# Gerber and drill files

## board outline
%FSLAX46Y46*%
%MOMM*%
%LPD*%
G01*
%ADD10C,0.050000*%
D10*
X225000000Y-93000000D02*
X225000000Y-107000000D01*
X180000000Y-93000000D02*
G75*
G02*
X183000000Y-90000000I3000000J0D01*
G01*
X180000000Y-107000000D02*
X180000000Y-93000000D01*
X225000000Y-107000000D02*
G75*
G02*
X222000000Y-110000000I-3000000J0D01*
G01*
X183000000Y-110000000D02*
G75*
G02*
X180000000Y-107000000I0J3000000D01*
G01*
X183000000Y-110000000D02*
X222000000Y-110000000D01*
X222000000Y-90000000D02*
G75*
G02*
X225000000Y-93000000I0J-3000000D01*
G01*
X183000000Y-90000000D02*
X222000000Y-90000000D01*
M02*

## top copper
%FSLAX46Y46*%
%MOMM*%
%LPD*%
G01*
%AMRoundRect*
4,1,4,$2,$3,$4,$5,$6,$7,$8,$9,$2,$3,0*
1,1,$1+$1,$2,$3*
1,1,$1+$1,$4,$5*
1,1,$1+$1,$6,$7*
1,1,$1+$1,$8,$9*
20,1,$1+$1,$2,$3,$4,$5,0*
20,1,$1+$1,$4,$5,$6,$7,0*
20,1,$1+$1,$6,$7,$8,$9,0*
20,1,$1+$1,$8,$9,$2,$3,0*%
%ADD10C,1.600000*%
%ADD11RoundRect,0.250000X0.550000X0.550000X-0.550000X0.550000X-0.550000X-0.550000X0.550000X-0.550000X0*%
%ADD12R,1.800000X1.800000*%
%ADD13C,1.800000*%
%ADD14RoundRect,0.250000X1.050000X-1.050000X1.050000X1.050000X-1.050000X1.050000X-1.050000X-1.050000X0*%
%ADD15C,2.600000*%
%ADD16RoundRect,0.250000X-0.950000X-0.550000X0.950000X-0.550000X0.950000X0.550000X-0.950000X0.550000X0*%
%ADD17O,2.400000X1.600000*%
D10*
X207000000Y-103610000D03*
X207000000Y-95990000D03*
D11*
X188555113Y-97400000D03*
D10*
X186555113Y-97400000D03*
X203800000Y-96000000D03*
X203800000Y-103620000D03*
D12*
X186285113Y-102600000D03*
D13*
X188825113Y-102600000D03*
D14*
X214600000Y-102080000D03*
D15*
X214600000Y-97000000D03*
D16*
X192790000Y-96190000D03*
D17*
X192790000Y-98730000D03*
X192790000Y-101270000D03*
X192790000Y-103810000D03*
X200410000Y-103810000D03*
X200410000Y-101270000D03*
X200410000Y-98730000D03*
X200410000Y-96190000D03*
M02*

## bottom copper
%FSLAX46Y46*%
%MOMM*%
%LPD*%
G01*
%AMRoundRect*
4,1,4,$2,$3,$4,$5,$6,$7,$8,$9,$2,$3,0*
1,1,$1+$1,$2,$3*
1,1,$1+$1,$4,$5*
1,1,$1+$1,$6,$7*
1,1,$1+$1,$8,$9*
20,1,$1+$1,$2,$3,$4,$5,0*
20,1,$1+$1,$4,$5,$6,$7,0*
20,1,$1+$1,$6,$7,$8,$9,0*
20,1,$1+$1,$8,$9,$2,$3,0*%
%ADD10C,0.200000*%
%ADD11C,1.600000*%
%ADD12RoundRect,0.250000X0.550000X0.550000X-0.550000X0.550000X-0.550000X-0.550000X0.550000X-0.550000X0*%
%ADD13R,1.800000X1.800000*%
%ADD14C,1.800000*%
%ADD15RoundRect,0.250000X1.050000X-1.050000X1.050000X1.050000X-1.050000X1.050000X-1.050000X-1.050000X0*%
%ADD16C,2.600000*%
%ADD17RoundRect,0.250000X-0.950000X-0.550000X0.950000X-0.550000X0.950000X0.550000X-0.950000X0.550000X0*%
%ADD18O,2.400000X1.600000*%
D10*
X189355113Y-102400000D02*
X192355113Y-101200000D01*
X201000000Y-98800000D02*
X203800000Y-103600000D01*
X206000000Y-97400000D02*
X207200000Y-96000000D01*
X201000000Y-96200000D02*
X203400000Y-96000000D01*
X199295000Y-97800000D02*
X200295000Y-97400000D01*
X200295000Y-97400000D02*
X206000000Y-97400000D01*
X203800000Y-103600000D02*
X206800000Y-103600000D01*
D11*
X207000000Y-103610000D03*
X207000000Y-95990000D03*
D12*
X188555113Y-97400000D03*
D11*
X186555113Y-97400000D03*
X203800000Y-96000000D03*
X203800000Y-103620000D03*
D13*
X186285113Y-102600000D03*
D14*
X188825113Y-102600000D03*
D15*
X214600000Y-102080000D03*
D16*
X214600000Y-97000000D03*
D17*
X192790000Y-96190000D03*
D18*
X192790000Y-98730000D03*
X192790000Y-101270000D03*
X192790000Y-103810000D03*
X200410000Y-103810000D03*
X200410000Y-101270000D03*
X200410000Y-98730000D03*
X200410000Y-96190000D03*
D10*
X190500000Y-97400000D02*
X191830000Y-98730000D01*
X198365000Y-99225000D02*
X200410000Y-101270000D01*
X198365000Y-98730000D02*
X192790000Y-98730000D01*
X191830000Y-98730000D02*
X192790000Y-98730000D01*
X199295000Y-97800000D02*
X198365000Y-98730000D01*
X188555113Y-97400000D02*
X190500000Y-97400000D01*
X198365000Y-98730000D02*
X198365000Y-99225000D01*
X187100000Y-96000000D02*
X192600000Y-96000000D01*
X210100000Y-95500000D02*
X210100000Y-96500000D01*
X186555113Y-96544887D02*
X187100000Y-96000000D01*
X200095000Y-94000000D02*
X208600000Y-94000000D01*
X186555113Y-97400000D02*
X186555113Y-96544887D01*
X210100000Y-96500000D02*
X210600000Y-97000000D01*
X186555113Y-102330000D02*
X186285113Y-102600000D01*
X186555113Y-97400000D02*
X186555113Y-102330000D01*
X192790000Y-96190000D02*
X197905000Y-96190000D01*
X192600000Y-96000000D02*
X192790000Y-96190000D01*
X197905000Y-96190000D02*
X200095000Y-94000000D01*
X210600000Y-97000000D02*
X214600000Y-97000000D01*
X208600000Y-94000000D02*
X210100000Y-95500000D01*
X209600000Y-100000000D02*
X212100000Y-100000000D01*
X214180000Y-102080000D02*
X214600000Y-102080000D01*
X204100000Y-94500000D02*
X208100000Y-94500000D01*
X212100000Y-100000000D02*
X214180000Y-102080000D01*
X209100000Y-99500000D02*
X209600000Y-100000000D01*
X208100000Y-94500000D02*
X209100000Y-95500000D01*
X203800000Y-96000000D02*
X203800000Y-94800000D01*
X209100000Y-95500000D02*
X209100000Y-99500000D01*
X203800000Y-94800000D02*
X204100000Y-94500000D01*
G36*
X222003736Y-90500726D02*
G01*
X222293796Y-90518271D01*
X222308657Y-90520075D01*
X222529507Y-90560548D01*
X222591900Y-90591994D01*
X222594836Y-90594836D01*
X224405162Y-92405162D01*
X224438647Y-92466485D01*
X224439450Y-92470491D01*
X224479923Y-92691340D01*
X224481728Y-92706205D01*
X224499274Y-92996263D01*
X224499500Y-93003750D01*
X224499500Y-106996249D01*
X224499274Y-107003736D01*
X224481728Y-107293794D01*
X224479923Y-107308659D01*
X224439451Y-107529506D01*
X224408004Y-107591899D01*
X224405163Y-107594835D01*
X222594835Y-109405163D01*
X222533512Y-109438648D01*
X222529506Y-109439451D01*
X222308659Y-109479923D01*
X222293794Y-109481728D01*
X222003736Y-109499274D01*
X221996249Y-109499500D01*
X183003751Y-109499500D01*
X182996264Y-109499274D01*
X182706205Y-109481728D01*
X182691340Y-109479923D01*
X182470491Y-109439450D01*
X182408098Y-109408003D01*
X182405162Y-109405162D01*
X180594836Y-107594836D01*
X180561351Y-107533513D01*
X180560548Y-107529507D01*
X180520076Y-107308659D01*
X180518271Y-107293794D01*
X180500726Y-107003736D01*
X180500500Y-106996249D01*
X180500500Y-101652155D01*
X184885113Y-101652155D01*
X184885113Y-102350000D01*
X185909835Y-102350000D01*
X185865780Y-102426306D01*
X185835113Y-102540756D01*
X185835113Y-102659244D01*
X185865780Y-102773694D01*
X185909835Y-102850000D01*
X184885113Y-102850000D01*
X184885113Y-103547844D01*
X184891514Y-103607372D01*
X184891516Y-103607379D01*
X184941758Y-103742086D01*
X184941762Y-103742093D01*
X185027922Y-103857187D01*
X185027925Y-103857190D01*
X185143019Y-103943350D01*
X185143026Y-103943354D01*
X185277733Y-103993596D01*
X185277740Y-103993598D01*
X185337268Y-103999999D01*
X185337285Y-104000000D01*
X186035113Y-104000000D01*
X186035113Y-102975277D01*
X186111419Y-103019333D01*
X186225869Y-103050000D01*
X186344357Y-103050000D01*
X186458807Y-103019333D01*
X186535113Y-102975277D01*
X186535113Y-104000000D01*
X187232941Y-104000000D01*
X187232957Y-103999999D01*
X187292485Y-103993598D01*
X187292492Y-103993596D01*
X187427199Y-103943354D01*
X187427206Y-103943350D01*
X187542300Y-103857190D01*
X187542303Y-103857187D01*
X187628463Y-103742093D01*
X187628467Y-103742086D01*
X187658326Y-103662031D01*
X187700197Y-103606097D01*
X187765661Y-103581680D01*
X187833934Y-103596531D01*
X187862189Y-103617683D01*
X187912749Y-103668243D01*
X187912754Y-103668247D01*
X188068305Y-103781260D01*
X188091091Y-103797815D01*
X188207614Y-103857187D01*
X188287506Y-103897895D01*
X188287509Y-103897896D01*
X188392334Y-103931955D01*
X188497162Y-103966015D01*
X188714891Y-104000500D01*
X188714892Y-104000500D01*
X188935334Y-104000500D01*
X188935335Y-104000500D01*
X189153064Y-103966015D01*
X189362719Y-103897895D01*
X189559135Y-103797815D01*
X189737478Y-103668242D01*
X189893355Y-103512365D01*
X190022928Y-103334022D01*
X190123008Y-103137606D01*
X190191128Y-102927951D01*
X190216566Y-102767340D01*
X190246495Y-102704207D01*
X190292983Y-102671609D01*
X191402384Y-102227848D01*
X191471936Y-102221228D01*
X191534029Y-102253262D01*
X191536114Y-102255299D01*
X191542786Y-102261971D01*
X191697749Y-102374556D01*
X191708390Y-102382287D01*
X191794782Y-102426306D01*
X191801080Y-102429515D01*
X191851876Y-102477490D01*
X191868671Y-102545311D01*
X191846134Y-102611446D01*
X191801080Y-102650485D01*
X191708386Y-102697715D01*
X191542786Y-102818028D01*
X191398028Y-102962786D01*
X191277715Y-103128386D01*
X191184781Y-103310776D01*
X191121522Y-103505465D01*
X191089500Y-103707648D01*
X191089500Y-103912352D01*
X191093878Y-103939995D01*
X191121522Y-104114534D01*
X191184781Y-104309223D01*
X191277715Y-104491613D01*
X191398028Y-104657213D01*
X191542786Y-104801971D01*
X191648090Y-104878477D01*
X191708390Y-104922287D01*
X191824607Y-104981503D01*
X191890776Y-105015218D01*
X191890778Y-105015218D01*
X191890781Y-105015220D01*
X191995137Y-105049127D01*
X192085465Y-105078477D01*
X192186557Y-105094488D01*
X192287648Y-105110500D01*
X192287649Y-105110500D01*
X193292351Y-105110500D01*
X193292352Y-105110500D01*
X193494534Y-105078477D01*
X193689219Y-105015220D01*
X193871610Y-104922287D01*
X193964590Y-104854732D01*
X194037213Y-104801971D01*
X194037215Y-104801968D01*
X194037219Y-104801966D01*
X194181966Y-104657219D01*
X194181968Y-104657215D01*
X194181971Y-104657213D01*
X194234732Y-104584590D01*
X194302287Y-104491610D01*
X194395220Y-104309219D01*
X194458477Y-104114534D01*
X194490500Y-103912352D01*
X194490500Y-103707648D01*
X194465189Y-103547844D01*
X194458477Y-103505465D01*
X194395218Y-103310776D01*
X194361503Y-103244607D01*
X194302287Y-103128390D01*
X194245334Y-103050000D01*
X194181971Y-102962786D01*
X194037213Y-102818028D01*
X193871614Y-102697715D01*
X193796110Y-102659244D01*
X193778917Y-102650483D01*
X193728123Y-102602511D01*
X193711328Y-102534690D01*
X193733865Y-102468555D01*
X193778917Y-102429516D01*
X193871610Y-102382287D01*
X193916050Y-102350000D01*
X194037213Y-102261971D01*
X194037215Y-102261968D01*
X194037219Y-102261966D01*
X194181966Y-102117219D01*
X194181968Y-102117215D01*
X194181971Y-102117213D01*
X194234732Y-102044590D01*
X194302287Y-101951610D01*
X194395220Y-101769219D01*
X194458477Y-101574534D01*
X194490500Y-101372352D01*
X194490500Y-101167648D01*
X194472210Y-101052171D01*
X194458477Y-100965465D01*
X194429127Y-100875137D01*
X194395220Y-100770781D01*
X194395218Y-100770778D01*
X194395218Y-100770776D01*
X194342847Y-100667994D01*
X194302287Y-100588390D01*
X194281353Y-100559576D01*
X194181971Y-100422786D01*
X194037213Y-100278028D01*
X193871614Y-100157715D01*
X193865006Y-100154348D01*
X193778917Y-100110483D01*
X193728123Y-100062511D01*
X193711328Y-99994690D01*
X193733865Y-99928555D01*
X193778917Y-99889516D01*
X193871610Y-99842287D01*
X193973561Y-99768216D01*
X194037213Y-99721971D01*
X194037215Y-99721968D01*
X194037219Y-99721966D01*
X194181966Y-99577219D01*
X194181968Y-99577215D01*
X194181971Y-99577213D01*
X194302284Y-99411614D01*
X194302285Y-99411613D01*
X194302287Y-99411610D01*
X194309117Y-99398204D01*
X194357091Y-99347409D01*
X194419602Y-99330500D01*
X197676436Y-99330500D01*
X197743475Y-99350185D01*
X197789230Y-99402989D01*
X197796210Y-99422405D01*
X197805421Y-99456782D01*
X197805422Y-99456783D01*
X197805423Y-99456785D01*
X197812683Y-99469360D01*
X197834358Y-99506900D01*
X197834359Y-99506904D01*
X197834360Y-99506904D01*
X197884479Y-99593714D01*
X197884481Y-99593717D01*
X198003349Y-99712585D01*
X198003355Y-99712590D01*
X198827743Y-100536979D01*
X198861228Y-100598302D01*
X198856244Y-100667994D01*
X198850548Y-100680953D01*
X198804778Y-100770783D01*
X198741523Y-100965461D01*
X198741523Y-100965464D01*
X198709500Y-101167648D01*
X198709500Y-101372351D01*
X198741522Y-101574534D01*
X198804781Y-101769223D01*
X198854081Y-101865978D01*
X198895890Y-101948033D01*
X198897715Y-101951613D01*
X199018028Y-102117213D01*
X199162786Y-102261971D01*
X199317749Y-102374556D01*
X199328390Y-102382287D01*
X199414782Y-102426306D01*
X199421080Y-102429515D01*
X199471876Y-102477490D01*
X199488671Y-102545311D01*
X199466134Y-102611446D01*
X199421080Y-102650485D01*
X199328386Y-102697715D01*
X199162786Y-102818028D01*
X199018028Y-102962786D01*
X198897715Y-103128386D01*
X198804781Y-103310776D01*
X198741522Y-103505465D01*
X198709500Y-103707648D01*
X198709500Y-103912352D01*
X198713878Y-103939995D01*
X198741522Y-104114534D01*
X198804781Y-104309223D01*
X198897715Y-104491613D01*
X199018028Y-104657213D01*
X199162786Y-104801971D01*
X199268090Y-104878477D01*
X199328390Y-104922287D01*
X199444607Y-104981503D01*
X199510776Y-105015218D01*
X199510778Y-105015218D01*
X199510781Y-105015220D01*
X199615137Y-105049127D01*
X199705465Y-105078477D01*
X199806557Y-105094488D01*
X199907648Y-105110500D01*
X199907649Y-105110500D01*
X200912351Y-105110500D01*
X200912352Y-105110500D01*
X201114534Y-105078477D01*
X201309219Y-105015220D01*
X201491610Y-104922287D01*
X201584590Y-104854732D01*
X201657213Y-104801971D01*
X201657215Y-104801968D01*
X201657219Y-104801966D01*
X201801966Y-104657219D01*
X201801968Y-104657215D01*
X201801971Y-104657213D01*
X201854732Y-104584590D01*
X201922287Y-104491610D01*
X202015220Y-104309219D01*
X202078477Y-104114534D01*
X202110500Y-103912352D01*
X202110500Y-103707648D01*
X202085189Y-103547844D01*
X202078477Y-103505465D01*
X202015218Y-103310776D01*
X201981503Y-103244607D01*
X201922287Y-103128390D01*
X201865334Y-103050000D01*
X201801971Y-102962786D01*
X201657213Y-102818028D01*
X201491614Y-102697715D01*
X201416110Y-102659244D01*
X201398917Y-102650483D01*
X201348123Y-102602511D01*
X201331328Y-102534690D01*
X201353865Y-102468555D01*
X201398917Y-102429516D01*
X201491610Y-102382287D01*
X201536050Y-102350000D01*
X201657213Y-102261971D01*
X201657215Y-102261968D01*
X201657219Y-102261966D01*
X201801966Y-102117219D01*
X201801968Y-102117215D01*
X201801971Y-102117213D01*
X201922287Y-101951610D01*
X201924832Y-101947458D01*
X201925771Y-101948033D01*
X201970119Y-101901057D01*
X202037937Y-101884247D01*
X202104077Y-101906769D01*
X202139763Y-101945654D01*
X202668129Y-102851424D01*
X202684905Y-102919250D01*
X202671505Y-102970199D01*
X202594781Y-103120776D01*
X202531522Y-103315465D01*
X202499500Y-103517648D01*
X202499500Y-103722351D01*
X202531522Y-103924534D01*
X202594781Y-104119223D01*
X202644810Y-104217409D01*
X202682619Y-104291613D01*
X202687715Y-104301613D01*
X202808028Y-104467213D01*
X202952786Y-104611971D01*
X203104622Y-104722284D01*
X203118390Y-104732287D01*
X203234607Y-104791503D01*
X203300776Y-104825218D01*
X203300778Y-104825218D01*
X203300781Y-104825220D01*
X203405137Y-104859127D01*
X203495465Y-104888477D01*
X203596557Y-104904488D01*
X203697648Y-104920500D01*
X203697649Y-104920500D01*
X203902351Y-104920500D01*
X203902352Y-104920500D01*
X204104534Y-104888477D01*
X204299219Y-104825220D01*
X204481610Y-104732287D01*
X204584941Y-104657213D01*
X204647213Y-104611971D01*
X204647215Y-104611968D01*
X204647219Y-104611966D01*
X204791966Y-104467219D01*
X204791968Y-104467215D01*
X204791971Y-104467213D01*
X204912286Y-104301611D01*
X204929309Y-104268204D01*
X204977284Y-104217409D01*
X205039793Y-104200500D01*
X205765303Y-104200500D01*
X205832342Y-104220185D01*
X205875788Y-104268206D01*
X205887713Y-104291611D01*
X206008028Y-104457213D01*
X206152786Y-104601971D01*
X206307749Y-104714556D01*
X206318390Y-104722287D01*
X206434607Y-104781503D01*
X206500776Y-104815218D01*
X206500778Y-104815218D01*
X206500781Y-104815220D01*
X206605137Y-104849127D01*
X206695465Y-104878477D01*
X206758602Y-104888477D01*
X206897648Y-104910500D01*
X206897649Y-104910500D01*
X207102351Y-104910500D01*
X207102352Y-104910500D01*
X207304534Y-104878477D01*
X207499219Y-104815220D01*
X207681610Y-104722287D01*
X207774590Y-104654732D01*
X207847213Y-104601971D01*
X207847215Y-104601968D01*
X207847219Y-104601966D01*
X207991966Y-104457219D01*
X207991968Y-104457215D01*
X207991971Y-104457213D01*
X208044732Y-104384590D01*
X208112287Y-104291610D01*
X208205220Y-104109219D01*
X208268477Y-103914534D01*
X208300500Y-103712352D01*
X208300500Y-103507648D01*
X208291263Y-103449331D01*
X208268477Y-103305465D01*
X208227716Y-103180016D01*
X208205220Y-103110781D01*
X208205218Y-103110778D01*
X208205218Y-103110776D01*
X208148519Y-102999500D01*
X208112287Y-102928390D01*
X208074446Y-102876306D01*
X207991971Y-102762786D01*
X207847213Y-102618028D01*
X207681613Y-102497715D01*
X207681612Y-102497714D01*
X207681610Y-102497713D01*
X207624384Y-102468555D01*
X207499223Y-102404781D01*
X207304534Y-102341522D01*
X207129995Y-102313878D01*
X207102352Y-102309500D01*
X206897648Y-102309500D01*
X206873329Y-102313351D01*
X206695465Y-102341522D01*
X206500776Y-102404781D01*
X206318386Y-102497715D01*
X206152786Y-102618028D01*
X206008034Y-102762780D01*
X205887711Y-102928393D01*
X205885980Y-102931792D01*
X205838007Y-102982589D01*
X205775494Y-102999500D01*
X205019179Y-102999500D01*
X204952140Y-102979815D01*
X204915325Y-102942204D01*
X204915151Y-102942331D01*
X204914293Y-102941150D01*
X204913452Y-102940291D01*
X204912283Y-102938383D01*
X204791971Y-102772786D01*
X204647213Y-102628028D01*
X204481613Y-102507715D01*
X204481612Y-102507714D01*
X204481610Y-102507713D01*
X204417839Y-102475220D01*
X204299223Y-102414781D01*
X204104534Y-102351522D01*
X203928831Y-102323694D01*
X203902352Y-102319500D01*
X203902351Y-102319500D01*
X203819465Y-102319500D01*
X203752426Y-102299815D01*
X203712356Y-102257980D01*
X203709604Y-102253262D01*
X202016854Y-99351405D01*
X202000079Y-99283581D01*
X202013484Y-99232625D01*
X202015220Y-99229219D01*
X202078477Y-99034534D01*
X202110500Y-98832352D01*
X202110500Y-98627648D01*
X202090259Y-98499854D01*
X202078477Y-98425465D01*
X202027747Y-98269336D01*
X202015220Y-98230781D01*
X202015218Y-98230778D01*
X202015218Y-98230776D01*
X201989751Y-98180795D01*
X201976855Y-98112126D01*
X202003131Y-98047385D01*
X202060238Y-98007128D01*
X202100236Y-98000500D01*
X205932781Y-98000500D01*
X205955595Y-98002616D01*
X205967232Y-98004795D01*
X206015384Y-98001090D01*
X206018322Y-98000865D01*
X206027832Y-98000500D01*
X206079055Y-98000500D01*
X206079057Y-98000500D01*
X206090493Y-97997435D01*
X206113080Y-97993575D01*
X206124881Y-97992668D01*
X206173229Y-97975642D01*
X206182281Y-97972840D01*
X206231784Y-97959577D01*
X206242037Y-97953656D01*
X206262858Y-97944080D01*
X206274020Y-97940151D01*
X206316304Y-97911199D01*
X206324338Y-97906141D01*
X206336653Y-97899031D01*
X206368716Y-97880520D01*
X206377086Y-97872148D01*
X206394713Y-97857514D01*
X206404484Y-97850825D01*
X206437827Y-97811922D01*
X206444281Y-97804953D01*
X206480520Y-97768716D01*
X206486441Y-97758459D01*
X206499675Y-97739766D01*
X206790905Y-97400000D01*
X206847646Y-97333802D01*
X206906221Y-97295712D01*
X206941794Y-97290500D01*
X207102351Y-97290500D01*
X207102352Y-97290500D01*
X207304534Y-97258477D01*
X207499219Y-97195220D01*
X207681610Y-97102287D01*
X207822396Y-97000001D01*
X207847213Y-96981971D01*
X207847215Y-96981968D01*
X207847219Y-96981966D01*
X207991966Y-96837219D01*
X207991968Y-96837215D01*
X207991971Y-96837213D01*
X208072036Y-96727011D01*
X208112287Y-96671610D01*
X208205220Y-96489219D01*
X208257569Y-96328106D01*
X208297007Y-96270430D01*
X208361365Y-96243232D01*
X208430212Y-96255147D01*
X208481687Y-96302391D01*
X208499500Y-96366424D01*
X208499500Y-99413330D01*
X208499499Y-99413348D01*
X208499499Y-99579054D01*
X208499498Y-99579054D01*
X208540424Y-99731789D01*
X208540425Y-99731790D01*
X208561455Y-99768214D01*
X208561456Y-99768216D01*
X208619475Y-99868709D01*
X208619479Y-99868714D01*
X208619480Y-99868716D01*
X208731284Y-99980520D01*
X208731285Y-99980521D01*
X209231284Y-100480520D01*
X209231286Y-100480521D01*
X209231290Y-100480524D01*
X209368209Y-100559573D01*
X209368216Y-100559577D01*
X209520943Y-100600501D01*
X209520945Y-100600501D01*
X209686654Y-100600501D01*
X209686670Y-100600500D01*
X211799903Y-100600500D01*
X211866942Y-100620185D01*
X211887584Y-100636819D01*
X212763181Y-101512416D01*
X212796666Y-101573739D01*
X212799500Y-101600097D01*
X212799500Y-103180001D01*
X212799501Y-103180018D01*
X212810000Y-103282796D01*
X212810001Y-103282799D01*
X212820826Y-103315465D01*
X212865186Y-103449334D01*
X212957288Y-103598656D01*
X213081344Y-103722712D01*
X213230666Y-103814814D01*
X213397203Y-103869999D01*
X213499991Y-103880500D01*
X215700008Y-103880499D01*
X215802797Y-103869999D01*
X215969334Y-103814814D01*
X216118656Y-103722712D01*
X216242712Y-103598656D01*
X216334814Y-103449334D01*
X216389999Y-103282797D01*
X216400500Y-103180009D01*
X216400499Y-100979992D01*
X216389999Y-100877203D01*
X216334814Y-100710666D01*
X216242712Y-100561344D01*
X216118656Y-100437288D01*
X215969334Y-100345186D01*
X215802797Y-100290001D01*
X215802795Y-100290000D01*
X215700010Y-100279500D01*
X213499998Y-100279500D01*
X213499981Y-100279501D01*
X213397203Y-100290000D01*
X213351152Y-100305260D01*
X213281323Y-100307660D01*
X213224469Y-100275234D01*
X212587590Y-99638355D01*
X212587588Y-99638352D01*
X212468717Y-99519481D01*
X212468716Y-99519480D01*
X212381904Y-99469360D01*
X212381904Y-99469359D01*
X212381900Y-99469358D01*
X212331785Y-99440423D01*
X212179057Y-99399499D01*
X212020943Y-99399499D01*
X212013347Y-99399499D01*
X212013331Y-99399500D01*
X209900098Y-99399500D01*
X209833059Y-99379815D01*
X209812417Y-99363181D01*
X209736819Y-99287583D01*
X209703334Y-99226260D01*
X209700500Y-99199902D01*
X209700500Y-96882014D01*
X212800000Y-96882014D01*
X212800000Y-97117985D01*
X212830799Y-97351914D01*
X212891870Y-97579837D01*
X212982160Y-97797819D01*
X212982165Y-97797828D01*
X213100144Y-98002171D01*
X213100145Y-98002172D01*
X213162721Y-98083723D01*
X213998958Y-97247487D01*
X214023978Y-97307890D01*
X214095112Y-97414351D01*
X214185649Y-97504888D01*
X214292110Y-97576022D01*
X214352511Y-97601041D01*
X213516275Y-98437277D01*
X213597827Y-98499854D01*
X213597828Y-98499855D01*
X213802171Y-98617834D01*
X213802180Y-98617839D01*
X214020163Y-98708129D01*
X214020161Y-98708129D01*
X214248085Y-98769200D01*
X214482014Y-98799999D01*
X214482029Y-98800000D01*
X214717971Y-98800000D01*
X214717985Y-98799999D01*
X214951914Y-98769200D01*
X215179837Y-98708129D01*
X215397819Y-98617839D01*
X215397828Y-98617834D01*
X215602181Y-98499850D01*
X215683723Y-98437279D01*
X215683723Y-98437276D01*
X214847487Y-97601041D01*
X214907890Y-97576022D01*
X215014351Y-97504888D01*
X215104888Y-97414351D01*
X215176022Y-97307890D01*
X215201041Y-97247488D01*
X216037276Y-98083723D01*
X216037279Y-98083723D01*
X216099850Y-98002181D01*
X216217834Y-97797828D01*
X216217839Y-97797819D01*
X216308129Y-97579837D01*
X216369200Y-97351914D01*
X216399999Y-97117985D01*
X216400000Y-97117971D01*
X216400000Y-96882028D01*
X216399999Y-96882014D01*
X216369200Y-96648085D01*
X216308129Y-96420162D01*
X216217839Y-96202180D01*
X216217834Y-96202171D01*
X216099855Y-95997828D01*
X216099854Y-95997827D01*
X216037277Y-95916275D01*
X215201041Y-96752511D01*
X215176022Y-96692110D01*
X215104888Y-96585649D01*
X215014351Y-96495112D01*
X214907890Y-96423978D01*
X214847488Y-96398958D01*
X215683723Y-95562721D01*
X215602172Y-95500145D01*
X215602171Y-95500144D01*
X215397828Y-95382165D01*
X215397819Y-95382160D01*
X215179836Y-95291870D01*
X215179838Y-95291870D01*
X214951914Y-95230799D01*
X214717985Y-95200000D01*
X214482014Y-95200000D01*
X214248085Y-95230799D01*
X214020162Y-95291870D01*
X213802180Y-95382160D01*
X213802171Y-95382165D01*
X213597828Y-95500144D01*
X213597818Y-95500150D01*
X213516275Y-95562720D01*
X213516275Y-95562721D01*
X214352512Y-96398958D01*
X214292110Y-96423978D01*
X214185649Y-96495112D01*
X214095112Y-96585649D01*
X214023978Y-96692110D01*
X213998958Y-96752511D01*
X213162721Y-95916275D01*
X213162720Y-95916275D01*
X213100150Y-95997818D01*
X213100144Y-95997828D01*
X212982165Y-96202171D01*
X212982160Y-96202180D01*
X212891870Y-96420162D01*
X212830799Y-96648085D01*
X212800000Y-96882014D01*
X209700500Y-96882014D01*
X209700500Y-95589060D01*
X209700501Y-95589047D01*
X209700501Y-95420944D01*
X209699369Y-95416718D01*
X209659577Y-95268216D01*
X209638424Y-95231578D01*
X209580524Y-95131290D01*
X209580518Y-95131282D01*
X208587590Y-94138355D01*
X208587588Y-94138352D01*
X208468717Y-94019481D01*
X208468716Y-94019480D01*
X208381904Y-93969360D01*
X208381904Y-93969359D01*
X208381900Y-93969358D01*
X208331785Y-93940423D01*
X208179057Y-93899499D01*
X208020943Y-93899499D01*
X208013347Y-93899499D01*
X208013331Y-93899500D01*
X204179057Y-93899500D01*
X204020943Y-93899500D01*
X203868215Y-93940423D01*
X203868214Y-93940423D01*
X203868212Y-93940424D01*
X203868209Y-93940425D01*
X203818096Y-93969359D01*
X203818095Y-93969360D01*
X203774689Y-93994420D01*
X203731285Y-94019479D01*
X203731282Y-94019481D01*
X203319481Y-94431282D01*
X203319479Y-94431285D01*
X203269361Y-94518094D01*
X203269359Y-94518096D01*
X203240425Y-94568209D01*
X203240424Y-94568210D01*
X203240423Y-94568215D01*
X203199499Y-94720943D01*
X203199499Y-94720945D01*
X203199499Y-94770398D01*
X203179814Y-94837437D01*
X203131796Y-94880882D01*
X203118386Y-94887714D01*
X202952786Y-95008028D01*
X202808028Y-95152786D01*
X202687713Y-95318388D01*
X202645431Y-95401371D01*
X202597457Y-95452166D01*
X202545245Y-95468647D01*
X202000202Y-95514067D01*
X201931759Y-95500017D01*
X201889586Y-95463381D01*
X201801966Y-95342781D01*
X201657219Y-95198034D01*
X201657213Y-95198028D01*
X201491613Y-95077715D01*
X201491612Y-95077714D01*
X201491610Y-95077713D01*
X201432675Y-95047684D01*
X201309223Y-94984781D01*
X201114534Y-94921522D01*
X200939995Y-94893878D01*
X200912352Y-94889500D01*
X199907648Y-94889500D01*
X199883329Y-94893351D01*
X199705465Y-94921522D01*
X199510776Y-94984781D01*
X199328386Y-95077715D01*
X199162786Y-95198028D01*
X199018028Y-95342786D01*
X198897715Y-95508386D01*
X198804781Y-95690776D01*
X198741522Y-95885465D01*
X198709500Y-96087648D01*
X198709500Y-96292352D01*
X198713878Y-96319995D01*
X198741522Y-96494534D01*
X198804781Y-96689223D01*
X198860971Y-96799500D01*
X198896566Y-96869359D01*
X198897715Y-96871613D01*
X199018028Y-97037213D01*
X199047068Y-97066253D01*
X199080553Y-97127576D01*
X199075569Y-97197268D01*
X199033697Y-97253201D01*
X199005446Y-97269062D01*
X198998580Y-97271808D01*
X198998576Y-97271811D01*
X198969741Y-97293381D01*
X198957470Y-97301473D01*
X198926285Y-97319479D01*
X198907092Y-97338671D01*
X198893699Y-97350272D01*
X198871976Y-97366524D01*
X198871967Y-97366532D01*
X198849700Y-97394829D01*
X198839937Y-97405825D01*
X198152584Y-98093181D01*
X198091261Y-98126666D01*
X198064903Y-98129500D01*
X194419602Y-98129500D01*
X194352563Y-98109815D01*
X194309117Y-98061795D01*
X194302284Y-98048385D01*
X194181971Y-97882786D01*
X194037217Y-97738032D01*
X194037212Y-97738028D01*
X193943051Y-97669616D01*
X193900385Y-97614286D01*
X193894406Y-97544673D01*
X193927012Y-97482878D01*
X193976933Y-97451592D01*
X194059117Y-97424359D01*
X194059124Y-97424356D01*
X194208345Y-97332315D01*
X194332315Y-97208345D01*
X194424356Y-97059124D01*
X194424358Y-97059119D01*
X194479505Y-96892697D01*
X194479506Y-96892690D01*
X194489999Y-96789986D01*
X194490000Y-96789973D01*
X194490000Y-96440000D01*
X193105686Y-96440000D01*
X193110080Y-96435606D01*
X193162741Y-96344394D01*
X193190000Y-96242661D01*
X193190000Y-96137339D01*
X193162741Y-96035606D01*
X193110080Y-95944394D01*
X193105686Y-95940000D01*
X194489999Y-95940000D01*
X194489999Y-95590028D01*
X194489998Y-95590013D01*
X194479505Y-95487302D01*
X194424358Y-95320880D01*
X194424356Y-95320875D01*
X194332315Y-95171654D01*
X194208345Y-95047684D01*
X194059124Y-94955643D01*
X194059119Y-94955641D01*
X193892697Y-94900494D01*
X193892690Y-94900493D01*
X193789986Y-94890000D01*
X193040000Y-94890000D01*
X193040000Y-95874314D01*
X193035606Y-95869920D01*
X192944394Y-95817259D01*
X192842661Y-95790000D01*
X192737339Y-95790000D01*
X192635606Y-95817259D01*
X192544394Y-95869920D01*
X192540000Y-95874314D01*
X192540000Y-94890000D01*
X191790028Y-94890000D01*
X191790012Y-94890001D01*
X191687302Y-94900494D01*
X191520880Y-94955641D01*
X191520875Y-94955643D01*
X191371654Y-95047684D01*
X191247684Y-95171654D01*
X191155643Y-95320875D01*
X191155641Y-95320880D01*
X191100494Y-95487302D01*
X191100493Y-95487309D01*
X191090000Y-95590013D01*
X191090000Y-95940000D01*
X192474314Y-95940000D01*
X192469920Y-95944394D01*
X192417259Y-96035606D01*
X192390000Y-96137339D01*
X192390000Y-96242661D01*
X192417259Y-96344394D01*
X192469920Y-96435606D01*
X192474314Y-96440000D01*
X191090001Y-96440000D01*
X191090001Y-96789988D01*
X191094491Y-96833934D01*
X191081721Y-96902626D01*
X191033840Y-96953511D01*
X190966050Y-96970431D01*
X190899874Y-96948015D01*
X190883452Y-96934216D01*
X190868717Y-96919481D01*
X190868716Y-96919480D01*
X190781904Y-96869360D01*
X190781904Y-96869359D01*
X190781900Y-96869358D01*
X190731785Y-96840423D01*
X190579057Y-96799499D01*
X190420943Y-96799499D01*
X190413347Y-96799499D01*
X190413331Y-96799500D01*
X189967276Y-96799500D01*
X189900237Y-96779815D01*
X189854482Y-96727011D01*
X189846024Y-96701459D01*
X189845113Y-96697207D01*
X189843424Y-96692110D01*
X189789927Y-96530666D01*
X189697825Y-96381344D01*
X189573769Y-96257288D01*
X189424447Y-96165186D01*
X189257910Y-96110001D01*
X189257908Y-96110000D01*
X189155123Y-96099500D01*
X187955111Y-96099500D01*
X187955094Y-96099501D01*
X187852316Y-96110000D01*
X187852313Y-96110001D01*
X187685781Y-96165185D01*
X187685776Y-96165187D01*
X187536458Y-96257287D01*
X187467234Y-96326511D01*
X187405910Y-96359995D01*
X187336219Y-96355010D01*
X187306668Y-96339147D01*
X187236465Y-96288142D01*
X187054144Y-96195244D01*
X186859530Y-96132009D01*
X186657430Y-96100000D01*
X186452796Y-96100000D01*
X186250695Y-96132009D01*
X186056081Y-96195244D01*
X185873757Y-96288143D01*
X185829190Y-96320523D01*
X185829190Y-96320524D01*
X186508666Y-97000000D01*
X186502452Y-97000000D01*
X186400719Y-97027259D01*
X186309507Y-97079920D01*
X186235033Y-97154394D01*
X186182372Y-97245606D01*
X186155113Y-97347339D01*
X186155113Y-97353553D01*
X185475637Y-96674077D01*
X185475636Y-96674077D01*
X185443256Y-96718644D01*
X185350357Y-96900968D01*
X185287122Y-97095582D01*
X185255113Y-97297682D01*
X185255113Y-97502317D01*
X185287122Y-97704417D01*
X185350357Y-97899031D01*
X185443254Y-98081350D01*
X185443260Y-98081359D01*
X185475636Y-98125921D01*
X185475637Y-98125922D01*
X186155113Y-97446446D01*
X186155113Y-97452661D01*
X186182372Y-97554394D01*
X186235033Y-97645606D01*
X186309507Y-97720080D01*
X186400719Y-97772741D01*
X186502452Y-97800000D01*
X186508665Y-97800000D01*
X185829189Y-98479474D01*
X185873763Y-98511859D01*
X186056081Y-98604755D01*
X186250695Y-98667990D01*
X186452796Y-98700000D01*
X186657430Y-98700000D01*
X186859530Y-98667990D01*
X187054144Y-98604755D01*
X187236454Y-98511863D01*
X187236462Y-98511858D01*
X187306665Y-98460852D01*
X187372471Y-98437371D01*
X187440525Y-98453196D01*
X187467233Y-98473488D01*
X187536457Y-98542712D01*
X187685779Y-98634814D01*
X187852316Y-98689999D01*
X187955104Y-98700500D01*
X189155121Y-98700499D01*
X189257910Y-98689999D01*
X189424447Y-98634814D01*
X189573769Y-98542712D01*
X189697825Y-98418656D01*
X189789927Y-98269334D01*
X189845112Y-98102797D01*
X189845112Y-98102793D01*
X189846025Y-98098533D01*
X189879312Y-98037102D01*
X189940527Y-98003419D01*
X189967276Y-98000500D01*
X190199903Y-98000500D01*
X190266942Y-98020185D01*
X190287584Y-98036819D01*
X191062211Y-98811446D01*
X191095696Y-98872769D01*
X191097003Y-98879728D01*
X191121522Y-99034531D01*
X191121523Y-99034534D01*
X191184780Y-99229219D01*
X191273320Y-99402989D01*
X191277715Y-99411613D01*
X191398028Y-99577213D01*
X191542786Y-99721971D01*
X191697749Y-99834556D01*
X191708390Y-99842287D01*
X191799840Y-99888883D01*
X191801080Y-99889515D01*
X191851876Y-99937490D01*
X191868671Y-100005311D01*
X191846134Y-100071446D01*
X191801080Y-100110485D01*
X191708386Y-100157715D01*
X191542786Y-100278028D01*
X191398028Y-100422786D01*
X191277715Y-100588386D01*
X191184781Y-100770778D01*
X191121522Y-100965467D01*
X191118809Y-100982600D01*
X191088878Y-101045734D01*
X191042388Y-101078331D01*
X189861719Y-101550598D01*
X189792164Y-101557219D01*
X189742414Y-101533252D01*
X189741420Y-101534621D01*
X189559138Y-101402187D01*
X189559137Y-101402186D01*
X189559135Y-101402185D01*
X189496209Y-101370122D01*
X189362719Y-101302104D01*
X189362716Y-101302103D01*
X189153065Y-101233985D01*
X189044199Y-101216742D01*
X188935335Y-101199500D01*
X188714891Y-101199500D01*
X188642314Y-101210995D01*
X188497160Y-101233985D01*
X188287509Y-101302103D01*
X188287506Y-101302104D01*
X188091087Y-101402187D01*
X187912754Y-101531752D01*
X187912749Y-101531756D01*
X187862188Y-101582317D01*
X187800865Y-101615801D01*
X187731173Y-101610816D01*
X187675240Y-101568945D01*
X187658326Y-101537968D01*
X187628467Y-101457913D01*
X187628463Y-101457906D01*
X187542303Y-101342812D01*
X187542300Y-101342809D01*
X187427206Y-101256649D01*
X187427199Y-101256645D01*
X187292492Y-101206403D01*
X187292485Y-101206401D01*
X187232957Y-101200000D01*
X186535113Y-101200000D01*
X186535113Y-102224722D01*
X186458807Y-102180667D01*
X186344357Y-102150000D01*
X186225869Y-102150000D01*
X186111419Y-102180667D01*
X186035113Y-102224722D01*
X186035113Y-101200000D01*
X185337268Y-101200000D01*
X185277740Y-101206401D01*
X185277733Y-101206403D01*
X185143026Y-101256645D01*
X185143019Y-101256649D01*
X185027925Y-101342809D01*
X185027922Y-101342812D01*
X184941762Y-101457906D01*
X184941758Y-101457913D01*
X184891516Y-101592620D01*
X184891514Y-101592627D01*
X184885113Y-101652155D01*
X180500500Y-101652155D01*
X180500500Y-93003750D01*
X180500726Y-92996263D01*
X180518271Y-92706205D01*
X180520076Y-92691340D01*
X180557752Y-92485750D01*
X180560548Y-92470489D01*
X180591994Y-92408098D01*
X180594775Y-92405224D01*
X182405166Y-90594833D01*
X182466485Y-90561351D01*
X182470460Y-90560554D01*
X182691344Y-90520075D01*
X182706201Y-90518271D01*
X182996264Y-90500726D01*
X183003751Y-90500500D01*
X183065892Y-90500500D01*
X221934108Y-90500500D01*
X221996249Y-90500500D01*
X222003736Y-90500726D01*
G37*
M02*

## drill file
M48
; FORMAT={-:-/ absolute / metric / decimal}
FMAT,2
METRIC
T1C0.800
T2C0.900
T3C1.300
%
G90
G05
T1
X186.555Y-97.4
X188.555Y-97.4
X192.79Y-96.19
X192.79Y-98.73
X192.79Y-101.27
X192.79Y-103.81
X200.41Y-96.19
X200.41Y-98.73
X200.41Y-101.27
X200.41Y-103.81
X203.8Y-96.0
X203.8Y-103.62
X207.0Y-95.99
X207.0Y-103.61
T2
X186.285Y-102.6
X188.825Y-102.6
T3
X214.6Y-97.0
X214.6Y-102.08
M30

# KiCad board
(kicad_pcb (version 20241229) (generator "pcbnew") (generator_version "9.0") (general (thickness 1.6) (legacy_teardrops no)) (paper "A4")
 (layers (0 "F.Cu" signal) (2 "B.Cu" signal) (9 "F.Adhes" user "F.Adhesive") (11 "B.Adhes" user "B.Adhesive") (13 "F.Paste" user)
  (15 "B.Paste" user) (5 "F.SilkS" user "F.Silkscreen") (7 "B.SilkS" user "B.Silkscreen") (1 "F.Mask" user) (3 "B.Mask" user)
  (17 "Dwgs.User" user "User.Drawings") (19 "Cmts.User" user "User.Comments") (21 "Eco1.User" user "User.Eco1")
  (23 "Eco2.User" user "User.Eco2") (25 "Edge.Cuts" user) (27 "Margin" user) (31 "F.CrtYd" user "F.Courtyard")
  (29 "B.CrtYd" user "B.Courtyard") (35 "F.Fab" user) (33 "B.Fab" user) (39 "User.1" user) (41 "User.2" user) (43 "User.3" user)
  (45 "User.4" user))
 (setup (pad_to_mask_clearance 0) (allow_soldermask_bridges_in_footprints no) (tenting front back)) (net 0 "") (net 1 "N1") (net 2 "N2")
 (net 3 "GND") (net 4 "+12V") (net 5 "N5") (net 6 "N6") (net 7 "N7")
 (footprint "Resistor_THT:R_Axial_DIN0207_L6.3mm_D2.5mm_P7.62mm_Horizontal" (layer "F.Cu") (at 207 103.61 90)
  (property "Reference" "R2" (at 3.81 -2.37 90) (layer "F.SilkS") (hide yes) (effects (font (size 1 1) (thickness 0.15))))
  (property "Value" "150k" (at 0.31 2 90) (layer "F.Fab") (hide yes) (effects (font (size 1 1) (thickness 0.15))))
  (pad "1" thru_hole circle (at 0 0 90) (size 1.6 1.6) (drill 0.8) (layers "*.Cu" "*.Mask") (remove_unused_layers no) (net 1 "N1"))
  (pad "2" thru_hole circle (at 7.62 0 90) (size 1.6 1.6) (drill 0.8) (layers "*.Cu" "*.Mask") (remove_unused_layers no) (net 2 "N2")))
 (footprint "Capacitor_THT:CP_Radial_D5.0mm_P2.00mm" (layer "F.Cu") (at 188.555113 97.4 180)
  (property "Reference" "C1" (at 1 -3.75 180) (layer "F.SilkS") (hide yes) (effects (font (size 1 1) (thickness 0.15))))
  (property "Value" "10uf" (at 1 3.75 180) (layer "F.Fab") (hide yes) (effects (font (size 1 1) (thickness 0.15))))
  (pad "1" thru_hole roundrect (at 0 0 180) (size 1.6 1.6) (drill 0.8) (layers "*.Cu" "*.Mask") (remove_unused_layers no)
   (roundrect_rratio 0.15625) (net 2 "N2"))
  (pad "2" thru_hole circle (at 2 0 180) (size 1.6 1.6) (drill 0.8) (layers "*.Cu" "*.Mask") (remove_unused_layers no) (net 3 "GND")))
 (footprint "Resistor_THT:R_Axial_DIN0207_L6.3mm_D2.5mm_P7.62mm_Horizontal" (layer "F.Cu") (at 203.8 96 -90)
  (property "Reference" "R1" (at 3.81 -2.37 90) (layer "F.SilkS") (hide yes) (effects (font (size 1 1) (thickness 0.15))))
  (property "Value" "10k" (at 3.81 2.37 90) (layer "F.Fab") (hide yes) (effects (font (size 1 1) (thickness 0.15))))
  (pad "1" thru_hole circle (at 0 0 270) (size 1.6 1.6) (drill 0.8) (layers "*.Cu" "*.Mask") (remove_unused_layers no) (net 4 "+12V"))
  (pad "2" thru_hole circle (at 7.62 0 270) (size 1.6 1.6) (drill 0.8) (layers "*.Cu" "*.Mask") (remove_unused_layers no) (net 1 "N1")))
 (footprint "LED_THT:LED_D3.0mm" (layer "F.Cu") (at 186.285113 102.6)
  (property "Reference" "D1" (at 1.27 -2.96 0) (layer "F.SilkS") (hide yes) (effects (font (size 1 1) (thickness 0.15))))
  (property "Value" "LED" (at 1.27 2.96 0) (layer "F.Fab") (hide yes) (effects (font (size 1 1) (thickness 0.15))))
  (pad "1" thru_hole rect (at 0 0) (size 1.8 1.8) (drill 0.9) (layers "*.Cu" "*.Mask") (remove_unused_layers no) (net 3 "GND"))
  (pad "2" thru_hole circle (at 2.54 0) (size 1.8 1.8) (drill 0.9) (layers "*.Cu" "*.Mask") (remove_unused_layers no) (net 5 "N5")))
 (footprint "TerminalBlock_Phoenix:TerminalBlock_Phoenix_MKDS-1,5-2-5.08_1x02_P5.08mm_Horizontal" (layer "F.Cu") (at 214.6 102.08 90)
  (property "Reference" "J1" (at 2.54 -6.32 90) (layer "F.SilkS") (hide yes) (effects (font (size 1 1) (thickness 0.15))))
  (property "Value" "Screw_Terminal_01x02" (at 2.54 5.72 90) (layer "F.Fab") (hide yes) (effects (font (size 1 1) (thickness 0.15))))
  (pad "1" thru_hole roundrect (at 0 0 90) (size 2.6 2.6) (drill 1.3) (layers "*.Cu" "*.Mask") (remove_unused_layers no)
   (roundrect_rratio 0.096154) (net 4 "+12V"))
  (pad "2" thru_hole circle (at 5.08 0 90) (size 2.6 2.6) (drill 1.3) (layers "*.Cu" "*.Mask") (remove_unused_layers no) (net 3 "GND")))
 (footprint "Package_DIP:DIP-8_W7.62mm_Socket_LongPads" (layer "F.Cu") (at 192.79 96.19)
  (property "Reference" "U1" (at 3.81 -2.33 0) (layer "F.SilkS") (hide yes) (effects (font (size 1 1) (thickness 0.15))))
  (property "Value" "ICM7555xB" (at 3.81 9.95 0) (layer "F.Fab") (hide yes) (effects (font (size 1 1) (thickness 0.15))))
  (pad "1" thru_hole roundrect (at 0 0) (size 2.4 1.6) (drill 0.8) (layers "*.Cu" "*.Mask") (remove_unused_layers no)
   (roundrect_rratio 0.15625) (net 3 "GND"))
  (pad "2" thru_hole oval (at 0 2.54) (size 2.4 1.6) (drill 0.8) (layers "*.Cu" "*.Mask") (remove_unused_layers no) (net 2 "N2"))
  (pad "3" thru_hole oval (at 0 5.08) (size 2.4 1.6) (drill 0.8) (layers "*.Cu" "*.Mask") (remove_unused_layers no) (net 5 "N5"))
  (pad "4" thru_hole oval (at 0 7.62) (size 2.4 1.6) (drill 0.8) (layers "*.Cu" "*.Mask") (remove_unused_layers no) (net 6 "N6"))
  (pad "5" thru_hole oval (at 7.62 7.62) (size 2.4 1.6) (drill 0.8) (layers "*.Cu" "*.Mask") (remove_unused_layers no) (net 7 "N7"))
  (pad "6" thru_hole oval (at 7.62 5.08) (size 2.4 1.6) (drill 0.8) (layers "*.Cu" "*.Mask") (remove_unused_layers no) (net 2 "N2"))
  (pad "7" thru_hole oval (at 7.62 2.54) (size 2.4 1.6) (drill 0.8) (layers "*.Cu" "*.Mask") (remove_unused_layers no) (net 1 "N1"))
  (pad "8" thru_hole oval (at 7.62 0) (size 2.4 1.6) (drill 0.8) (layers "*.Cu" "*.Mask") (remove_unused_layers no) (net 4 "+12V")))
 (gr_line (start 189.355113 102.4) (end 192.355113 101.2) (stroke (width 0.2) (type default)) (layer "B.Cu") (net 5))
 (gr_line (start 201 98.8) (end 203.8 103.6) (stroke (width 0.2) (type default)) (layer "B.Cu") (net 1))
 (gr_line (start 206 97.4) (end 207.2 96) (stroke (width 0.2) (type default)) (layer "B.Cu") (net 2))
 (gr_line (start 201 96.2) (end 203.4 96) (stroke (width 0.2) (type default)) (layer "B.Cu") (net 4))
 (gr_line (start 199.295 97.8) (end 200.295 97.4) (stroke (width 0.2) (type default)) (layer "B.Cu") (net 2))
 (gr_line (start 200.295 97.4) (end 206 97.4) (stroke (width 0.2) (type default)) (layer "B.Cu") (net 2))
 (gr_line (start 203.8 103.6) (end 206.8 103.6) (stroke (width 0.2) (type default)) (layer "B.Cu") (net 1))
 (gr_line (start 225 93) (end 225 107) (stroke (width 0.05) (type default)) (layer "Edge.Cuts"))
 (gr_arc (start 180 93) (mid 180.87868 90.87868) (end 183 90) (stroke (width 0.05) (type default)) (layer "Edge.Cuts"))
 (gr_line (start 180 107) (end 180 93) (stroke (width 0.05) (type default)) (layer "Edge.Cuts"))
 (gr_arc (start 225 107) (mid 224.12132 109.12132) (end 222 110) (stroke (width 0.05) (type default)) (layer "Edge.Cuts"))
 (gr_arc (start 183 110) (mid 180.87868 109.12132) (end 180 107) (stroke (width 0.05) (type default)) (layer "Edge.Cuts"))
 (gr_line (start 183 110) (end 222 110) (stroke (width 0.05) (type default)) (layer "Edge.Cuts"))
 (gr_arc (start 222 90) (mid 224.12132 90.87868) (end 225 93) (stroke (width 0.05) (type default)) (layer "Edge.Cuts"))
 (gr_line (start 183 90) (end 222 90) (stroke (width 0.05) (type default)) (layer "Edge.Cuts"))
 (segment (start 190.5 97.4) (end 191.83 98.73) (width 0.2) (layer "B.Cu") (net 2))
 (segment (start 198.365 99.225) (end 200.41 101.27) (width 0.2) (layer "B.Cu") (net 2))
 (segment (start 198.365 98.73) (end 192.79 98.73) (width 0.2) (layer "B.Cu") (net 2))
 (segment (start 191.83 98.73) (end 192.79 98.73) (width 0.2) (layer "B.Cu") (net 2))
 (segment (start 199.295 97.8) (end 198.365 98.73) (width 0.2) (layer "B.Cu") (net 2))
 (segment (start 188.555113 97.4) (end 190.5 97.4) (width 0.2) (layer "B.Cu") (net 2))
 (segment (start 198.365 98.73) (end 198.365 99.225) (width 0.2) (layer "B.Cu") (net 2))
 (segment (start 187.1 96) (end 192.6 96) (width 0.2) (layer "B.Cu") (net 3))
 (segment (start 210.1 95.5) (end 210.1 96.5) (width 0.2) (layer "B.Cu") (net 3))
 (segment (start 186.555113 96.544887) (end 187.1 96) (width 0.2) (layer "B.Cu") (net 3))
 (segment (start 200.095 94) (end 208.6 94) (width 0.2) (layer "B.Cu") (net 3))
 (segment (start 186.555113 97.4) (end 186.555113 96.544887) (width 0.2) (layer "B.Cu") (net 3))
 (segment (start 210.1 96.5) (end 210.6 97) (width 0.2) (layer "B.Cu") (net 3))
 (segment (start 186.555113 102.33) (end 186.285113 102.6) (width 0.2) (layer "B.Cu") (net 3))
 (segment (start 186.555113 97.4) (end 186.555113 102.33) (width 0.2) (layer "B.Cu") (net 3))
 (segment (start 192.79 96.19) (end 197.905 96.19) (width 0.2) (layer "B.Cu") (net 3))
 (segment (start 192.6 96) (end 192.79 96.19) (width 0.2) (layer "B.Cu") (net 3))
 (segment (start 197.905 96.19) (end 200.095 94) (width 0.2) (layer "B.Cu") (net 3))
 (segment (start 210.6 97) (end 214.6 97) (width 0.2) (layer "B.Cu") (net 3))
 (segment (start 208.6 94) (end 210.1 95.5) (width 0.2) (layer "B.Cu") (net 3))
 (segment (start 209.6 100) (end 212.1 100) (width 0.2) (layer "B.Cu") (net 4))
 (segment (start 214.18 102.08) (end 214.6 102.08) (width 0.2) (layer "B.Cu") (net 4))
 (segment (start 204.1 94.5) (end 208.1 94.5) (width 0.2) (layer "B.Cu") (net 4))
 (segment (start 212.1 100) (end 214.18 102.08) (width 0.2) (layer "B.Cu") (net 4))
 (segment (start 209.1 99.5) (end 209.6 100) (width 0.2) (layer "B.Cu") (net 4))
 (segment (start 208.1 94.5) (end 209.1 95.5) (width 0.2) (layer "B.Cu") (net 4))
 (segment (start 203.8 96) (end 203.8 94.8) (width 0.2) (layer "B.Cu") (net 4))
 (segment (start 209.1 95.5) (end 209.1 99.5) (width 0.2) (layer "B.Cu") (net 4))
 (segment (start 203.8 94.8) (end 204.1 94.5) (width 0.2) (layer "B.Cu") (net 4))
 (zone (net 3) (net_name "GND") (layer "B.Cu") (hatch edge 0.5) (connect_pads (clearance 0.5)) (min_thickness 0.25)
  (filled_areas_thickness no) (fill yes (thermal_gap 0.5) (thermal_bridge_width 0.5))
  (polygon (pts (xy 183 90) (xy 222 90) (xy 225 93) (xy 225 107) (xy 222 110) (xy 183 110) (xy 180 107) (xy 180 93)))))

